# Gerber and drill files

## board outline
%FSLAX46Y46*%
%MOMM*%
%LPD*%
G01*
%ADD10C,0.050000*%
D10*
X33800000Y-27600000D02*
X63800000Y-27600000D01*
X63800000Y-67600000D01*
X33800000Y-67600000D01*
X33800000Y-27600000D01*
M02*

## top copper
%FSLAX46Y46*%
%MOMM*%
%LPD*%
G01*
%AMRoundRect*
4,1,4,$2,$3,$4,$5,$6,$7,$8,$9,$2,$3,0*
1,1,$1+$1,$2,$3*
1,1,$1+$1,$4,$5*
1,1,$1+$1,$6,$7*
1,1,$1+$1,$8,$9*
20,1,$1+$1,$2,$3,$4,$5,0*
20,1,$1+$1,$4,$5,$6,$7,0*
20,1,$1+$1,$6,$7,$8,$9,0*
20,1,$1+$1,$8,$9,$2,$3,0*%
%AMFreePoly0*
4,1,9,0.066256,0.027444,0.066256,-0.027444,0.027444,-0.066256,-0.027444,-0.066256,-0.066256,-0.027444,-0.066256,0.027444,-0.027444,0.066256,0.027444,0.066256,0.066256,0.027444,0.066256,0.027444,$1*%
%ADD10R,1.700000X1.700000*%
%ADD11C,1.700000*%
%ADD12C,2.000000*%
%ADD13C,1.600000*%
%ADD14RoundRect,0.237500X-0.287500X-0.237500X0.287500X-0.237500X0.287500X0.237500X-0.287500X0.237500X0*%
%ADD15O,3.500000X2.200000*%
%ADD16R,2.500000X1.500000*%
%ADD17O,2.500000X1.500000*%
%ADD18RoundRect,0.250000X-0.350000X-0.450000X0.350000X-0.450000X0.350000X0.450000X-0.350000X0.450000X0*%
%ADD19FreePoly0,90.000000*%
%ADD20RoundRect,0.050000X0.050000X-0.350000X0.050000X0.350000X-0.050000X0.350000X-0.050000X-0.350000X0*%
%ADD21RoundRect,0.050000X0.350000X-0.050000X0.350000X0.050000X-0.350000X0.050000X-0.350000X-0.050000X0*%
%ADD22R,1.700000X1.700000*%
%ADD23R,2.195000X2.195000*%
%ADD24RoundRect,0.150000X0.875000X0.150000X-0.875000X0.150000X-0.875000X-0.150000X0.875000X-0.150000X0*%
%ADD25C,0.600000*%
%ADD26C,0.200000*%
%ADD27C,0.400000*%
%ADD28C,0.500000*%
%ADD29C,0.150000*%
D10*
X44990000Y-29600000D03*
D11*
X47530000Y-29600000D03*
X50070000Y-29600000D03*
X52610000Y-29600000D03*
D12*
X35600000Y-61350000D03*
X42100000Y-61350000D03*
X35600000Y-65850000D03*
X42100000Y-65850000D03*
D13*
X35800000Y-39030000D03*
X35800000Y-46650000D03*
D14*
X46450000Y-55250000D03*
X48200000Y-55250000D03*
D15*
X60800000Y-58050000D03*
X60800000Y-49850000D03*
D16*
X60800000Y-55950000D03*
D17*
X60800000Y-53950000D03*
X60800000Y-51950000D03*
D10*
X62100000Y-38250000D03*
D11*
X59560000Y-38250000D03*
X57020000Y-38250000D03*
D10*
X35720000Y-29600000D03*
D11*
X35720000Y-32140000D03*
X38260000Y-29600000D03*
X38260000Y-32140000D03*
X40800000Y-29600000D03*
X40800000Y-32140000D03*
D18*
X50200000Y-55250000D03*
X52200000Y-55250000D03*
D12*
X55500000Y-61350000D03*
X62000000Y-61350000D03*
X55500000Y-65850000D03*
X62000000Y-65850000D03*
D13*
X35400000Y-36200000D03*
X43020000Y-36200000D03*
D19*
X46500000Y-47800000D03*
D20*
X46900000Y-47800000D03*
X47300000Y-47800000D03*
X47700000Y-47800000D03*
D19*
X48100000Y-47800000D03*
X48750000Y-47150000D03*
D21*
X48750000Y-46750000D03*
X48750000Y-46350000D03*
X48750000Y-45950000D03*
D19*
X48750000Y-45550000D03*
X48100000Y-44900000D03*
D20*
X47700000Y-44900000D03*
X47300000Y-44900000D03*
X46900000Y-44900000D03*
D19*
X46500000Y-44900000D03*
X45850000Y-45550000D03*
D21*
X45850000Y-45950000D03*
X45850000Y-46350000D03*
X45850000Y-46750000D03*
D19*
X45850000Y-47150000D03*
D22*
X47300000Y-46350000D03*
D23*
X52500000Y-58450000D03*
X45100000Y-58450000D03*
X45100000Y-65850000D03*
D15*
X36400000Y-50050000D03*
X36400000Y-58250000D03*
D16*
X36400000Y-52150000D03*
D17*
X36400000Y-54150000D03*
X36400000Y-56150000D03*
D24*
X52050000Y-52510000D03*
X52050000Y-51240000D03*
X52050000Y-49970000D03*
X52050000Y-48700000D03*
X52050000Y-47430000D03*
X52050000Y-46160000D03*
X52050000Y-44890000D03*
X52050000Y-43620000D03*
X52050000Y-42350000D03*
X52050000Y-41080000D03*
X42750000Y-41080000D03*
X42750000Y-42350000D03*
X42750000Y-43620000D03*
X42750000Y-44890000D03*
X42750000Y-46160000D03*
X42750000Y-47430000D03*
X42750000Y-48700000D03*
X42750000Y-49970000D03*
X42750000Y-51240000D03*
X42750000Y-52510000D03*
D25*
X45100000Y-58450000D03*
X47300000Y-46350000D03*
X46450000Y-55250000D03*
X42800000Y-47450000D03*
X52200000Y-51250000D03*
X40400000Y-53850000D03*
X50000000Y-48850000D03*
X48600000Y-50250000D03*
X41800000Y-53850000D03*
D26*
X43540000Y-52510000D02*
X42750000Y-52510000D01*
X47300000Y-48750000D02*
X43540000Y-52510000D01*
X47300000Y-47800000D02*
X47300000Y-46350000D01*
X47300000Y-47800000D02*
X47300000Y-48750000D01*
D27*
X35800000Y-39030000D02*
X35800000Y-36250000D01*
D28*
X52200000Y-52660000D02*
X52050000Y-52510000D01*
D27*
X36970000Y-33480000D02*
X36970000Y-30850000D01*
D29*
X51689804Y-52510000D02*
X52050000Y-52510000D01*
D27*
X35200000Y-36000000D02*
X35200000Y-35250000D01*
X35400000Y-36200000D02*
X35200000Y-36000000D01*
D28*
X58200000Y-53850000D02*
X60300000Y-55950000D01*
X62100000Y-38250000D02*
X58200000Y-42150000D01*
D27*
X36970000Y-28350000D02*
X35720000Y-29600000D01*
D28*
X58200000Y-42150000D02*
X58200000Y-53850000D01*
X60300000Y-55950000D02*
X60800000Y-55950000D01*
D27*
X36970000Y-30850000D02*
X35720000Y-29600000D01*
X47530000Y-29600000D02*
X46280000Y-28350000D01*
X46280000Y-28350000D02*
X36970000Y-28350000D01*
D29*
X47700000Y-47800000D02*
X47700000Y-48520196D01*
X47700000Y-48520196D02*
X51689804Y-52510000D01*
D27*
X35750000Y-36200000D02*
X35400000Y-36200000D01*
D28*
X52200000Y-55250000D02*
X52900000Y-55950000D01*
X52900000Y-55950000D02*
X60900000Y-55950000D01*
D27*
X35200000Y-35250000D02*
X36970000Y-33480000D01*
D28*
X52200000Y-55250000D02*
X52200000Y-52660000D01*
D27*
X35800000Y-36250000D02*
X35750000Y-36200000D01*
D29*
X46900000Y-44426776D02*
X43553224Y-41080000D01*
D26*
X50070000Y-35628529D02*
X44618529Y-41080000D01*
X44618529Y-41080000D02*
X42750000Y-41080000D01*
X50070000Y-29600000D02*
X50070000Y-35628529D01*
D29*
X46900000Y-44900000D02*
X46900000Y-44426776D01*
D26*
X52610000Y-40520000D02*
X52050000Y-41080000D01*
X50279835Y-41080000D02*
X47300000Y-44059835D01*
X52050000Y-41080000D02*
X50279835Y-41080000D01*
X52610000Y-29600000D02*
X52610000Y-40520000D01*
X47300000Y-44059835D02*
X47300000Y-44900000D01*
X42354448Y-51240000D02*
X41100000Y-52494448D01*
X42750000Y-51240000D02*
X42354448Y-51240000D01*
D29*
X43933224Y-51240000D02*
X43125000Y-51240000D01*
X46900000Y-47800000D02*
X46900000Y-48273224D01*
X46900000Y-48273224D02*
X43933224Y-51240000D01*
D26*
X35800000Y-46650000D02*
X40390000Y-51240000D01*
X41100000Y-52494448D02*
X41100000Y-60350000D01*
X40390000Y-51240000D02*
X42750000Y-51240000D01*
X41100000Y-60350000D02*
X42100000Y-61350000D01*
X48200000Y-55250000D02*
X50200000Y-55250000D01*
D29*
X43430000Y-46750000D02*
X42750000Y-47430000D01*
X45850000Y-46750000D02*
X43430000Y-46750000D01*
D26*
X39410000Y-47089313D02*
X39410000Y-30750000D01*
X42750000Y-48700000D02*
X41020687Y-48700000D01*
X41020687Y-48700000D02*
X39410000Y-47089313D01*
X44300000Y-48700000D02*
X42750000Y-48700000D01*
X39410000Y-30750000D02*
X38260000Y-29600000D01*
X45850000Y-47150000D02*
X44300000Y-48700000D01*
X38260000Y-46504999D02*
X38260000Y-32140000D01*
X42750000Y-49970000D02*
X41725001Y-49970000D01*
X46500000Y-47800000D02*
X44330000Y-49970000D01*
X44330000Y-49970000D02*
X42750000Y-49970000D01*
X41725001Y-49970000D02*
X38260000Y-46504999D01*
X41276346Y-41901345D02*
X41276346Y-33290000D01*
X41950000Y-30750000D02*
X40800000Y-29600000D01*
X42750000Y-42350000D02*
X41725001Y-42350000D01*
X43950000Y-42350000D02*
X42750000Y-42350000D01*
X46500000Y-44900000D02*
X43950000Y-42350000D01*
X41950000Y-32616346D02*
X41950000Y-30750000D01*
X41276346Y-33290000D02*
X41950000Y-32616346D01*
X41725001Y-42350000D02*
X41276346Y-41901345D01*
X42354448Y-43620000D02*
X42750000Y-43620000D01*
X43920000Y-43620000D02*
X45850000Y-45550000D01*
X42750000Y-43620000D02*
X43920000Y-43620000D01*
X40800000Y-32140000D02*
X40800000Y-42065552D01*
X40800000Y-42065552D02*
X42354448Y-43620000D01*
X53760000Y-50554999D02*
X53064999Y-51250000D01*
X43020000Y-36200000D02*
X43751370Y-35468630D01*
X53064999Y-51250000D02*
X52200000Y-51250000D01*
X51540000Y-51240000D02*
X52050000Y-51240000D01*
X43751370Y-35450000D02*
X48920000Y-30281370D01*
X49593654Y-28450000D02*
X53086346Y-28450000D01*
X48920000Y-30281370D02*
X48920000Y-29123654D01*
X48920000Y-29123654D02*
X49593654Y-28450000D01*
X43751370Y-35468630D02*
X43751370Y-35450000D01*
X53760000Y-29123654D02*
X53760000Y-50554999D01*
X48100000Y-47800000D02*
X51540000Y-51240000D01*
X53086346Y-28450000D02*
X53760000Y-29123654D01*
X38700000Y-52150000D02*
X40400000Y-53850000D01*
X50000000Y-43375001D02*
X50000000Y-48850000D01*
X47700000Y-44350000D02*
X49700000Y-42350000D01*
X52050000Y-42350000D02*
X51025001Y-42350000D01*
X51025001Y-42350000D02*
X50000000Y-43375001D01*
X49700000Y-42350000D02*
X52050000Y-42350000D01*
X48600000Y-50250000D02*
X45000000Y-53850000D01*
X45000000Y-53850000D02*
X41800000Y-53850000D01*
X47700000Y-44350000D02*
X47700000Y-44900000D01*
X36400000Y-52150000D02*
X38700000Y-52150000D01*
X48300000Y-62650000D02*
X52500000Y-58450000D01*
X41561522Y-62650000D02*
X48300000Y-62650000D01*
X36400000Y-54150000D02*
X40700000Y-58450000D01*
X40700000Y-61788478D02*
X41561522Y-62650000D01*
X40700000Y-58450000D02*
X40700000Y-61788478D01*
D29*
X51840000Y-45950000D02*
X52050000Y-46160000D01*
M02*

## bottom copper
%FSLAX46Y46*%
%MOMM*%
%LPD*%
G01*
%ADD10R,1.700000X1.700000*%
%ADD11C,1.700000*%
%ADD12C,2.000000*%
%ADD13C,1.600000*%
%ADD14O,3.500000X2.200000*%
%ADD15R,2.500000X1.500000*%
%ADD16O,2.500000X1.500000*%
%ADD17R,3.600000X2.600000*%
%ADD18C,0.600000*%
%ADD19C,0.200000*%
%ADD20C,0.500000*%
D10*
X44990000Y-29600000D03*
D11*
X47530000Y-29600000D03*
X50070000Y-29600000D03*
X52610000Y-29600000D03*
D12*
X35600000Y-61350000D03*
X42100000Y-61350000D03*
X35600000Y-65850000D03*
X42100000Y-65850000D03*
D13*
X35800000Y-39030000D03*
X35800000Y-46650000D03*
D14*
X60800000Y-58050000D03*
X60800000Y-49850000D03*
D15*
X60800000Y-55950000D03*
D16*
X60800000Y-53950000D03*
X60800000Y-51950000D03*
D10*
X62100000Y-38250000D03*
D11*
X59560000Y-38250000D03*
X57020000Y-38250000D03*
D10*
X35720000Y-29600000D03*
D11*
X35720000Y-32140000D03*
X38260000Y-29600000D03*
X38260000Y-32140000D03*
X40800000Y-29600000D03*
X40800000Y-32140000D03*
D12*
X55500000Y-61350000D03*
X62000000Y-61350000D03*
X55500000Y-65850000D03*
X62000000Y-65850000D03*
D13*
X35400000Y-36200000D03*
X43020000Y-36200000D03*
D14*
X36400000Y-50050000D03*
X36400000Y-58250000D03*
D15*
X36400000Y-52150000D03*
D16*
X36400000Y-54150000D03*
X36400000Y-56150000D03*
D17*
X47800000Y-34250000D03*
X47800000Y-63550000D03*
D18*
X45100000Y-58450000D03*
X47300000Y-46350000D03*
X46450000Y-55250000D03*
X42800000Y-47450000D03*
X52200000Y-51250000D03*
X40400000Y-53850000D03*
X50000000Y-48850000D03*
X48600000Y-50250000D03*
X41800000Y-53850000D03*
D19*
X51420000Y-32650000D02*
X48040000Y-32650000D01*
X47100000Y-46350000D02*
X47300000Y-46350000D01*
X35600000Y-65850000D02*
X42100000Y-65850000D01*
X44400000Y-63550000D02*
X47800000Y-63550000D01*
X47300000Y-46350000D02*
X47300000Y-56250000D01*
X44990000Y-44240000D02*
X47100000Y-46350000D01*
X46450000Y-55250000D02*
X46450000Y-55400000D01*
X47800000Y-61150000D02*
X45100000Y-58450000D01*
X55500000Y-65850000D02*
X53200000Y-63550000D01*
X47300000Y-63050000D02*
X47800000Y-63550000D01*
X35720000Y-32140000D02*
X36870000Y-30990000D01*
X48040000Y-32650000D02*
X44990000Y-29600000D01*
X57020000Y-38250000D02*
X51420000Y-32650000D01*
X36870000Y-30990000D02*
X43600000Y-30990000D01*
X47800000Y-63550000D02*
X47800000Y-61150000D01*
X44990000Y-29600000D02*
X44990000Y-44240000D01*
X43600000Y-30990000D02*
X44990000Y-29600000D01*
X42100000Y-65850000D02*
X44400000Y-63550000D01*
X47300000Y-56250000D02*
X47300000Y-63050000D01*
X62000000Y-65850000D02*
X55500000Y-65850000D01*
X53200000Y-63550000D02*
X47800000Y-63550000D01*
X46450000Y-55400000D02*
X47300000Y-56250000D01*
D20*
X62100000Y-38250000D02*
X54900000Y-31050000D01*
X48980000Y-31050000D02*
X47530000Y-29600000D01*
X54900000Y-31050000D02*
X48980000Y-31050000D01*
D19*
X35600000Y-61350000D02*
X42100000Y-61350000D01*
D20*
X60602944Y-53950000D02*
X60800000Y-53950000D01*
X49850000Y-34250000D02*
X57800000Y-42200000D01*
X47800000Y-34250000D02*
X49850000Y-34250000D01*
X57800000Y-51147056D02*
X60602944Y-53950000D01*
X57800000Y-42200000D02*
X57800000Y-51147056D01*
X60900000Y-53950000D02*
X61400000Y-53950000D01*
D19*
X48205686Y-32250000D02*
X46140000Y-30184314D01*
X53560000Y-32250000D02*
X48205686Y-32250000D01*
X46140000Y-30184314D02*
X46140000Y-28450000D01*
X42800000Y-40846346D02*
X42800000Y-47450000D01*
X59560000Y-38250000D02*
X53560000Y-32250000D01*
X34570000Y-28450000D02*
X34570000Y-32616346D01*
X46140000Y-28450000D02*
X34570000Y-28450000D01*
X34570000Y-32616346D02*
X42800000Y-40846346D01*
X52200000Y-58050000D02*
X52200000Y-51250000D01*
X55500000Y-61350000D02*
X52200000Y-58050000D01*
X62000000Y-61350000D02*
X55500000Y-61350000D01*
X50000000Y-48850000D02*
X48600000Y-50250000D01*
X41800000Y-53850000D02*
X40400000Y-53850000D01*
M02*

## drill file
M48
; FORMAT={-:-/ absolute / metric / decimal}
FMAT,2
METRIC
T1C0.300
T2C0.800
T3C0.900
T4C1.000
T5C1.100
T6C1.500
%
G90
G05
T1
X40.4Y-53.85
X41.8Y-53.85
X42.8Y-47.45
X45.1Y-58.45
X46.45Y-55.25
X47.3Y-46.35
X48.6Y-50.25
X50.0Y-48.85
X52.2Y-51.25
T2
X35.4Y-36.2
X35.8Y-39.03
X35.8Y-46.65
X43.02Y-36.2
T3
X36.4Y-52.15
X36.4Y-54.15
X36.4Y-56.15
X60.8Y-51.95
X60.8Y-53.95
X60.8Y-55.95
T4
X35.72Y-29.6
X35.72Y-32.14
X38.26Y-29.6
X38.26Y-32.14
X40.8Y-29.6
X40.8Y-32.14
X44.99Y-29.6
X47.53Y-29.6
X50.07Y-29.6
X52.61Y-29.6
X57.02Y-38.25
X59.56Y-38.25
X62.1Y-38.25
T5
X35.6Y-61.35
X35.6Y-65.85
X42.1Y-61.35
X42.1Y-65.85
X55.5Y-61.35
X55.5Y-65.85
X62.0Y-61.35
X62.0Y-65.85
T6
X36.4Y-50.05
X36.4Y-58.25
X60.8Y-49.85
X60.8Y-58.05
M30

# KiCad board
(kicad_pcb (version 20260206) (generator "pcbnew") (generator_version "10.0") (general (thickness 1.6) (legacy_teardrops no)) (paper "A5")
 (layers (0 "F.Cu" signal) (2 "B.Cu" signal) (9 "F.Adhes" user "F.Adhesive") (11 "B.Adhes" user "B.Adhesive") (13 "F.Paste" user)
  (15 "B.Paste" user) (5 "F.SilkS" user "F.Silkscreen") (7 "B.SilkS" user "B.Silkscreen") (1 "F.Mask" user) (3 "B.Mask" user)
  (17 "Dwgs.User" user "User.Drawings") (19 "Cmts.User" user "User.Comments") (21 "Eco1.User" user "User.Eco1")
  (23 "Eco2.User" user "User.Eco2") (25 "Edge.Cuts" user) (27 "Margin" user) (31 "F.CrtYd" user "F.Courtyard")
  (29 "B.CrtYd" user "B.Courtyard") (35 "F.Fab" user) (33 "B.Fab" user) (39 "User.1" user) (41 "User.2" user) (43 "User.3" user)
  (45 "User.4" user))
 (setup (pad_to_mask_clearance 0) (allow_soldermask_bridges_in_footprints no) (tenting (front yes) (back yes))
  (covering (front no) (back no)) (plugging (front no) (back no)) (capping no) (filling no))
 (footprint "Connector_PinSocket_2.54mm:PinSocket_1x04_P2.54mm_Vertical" (layer "F.Cu") (at 44.99 29.6 90)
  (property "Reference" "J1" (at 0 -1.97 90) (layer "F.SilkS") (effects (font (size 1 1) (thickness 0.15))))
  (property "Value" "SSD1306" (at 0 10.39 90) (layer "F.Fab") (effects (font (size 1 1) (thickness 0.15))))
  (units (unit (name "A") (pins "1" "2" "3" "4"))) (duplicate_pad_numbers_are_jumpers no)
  (pad "1" thru_hole rect (at 0 0 90) (size 1.7 1.7) (drill 1) (layers "*.Cu" "*.Mask") (remove_unused_layers no) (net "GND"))
  (pad "2" thru_hole circle (at 0 2.54 90) (size 1.7 1.7) (drill 1) (layers "*.Cu" "*.Mask") (remove_unused_layers no) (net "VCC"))
  (pad "3" thru_hole circle (at 0 5.08 90) (size 1.7 1.7) (drill 1) (layers "*.Cu" "*.Mask") (remove_unused_layers no) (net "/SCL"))
  (pad "4" thru_hole circle (at 0 7.62 90) (size 1.7 1.7) (drill 1) (layers "*.Cu" "*.Mask") (remove_unused_layers no) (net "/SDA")))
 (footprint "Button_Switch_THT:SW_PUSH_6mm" (layer "F.Cu") (at 35.6 61.35)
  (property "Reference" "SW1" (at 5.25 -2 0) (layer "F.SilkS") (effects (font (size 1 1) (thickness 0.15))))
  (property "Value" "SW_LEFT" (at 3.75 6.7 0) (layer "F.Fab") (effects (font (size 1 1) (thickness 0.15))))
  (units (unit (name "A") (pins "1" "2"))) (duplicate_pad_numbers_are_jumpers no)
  (pad "1" thru_hole circle (at 0 0 90) (size 2 2) (drill 1.1) (layers "*.Cu" "*.Mask") (remove_unused_layers no) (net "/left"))
  (pad "1" thru_hole circle (at 6.5 0 90) (size 2 2) (drill 1.1) (layers "*.Cu" "*.Mask") (remove_unused_layers no) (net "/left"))
  (pad "2" thru_hole circle (at 0 4.5 90) (size 2 2) (drill 1.1) (layers "*.Cu" "*.Mask") (remove_unused_layers no) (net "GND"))
  (pad "2" thru_hole circle (at 6.5 4.5 90) (size 2 2) (drill 1.1) (layers "*.Cu" "*.Mask") (remove_unused_layers no) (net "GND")))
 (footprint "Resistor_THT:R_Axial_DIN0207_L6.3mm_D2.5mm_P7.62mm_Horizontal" (layer "F.Cu") (at 35.8 39.03 -90)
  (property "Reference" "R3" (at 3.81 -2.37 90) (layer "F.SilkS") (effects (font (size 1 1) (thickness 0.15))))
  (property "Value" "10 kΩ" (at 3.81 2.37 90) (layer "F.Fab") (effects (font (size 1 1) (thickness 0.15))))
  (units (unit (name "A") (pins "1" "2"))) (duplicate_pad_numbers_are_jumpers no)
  (pad "1" thru_hole circle (at 0 0 270) (size 1.6 1.6) (drill 0.8) (layers "*.Cu" "*.Mask") (remove_unused_layers no) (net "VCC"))
  (pad "2" thru_hole circle (at 7.62 0 270) (size 1.6 1.6) (drill 0.8) (layers "*.Cu" "*.Mask") (remove_unused_layers no) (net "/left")))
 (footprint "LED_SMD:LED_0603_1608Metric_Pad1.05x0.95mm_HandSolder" (layer "F.Cu") (at 47.325 55.25)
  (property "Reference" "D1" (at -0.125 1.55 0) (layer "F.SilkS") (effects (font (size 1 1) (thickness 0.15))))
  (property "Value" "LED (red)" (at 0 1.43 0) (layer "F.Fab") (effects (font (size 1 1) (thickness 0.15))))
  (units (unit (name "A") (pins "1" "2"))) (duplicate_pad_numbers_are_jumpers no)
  (pad "1" smd roundrect (at -0.875 0) (size 1.05 0.95) (layers "F.Cu" "F.Mask" "F.Paste") (roundrect_rratio 0.25) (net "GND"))
  (pad "2" smd roundrect (at 0.875 0) (size 1.05 0.95) (layers "F.Cu" "F.Mask" "F.Paste") (roundrect_rratio 0.25) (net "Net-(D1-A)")))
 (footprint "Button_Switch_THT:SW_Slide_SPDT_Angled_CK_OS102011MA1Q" (layer "F.Cu") (at 60.8 55.95 90)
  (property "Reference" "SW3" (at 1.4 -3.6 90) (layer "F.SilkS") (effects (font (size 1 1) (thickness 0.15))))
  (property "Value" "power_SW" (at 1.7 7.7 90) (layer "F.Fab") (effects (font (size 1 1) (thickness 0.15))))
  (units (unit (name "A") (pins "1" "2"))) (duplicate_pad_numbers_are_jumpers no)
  (pad "" thru_hole oval (at -2.1 0 90) (size 2.2 3.5) (drill 1.5) (layers "*.Cu" "*.Mask") (remove_unused_layers no))
  (pad "" thru_hole oval (at 6.1 0 90) (size 2.2 3.5) (drill 1.5) (layers "*.Cu" "*.Mask") (remove_unused_layers no))
  (pad "1" thru_hole rect (at 0 0 90) (size 1.5 2.5) (drill 0.9) (layers "*.Cu" "*.Mask") (remove_unused_layers no) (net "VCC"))
  (pad "2" thru_hole oval (at 2 0 90) (size 1.5 2.5) (drill 0.9) (layers "*.Cu" "*.Mask") (remove_unused_layers no) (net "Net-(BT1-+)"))
  (pad "3" thru_hole oval (at 4 0 90) (size 1.5 2.5) (drill 0.9) (layers "*.Cu" "*.Mask") (remove_unused_layers no)))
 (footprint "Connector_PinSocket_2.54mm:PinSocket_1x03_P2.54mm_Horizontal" (layer "F.Cu") (at 62.1 38.25 -90)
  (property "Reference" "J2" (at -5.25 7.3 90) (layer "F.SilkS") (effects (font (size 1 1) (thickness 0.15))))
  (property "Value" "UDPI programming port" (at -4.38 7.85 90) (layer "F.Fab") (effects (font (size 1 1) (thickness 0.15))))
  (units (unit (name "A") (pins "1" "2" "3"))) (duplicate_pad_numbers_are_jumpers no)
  (pad "1" thru_hole rect (at 0 0 270) (size 1.7 1.7) (drill 1) (layers "*.Cu" "*.Mask") (remove_unused_layers no) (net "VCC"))
  (pad "2" thru_hole circle (at 0 2.54 270) (size 1.7 1.7) (drill 1) (layers "*.Cu" "*.Mask") (remove_unused_layers no) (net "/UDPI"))
  (pad "3" thru_hole circle (at 0 5.08 270) (size 1.7 1.7) (drill 1) (layers "*.Cu" "*.Mask") (remove_unused_layers no) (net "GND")))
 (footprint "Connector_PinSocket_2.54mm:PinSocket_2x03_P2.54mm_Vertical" (layer "F.Cu") (at 35.72 29.6 90)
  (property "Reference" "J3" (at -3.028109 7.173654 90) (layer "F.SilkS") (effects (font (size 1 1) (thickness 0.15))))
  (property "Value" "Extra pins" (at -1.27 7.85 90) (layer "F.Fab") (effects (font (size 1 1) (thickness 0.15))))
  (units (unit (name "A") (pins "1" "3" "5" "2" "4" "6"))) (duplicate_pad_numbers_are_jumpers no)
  (pad "1" thru_hole rect (at 0 0 90) (size 1.7 1.7) (drill 1) (layers "*.Cu" "*.Mask") (remove_unused_layers no) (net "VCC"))
  (pad "2" thru_hole circle (at -2.54 0 90) (size 1.7 1.7) (drill 1) (layers "*.Cu" "*.Mask") (remove_unused_layers no) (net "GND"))
  (pad "3" thru_hole circle (at 0 2.54 90) (size 1.7 1.7) (drill 1) (layers "*.Cu" "*.Mask") (remove_unused_layers no) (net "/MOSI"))
  (pad "4" thru_hole circle (at -2.54 2.54 90) (size 1.7 1.7) (drill 1) (layers "*.Cu" "*.Mask") (remove_unused_layers no) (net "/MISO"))
  (pad "5" thru_hole circle (at 0 5.08 90) (size 1.7 1.7) (drill 1) (layers "*.Cu" "*.Mask") (remove_unused_layers no) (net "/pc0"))
  (pad "6" thru_hole circle (at -2.54 5.08 90) (size 1.7 1.7) (drill 1) (layers "*.Cu" "*.Mask") (remove_unused_layers no) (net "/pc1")))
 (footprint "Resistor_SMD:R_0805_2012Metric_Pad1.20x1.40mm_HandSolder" (layer "F.Cu") (at 51.2 55.25)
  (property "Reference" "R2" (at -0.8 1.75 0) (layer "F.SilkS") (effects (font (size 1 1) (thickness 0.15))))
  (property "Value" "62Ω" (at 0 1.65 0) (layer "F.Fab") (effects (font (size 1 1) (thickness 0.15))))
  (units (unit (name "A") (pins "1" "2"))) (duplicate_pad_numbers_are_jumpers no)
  (pad "1" smd roundrect (at -1 0) (size 1.2 1.4) (layers "F.Cu" "F.Mask" "F.Paste") (roundrect_rratio 0.208333) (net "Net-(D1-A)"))
  (pad "2" smd roundrect (at 1 0) (size 1.2 1.4) (layers "F.Cu" "F.Mask" "F.Paste") (roundrect_rratio 0.208333) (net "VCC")))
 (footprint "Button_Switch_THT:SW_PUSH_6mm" (layer "F.Cu") (at 55.5 61.35)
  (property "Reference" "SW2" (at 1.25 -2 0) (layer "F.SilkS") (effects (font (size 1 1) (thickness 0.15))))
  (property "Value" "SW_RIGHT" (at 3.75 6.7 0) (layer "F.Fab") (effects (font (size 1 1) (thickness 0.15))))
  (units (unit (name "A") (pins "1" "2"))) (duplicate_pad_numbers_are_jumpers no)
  (pad "1" thru_hole circle (at 0 0 90) (size 2 2) (drill 1.1) (layers "*.Cu" "*.Mask") (remove_unused_layers no) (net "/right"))
  (pad "1" thru_hole circle (at 6.5 0 90) (size 2 2) (drill 1.1) (layers "*.Cu" "*.Mask") (remove_unused_layers no) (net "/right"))
  (pad "2" thru_hole circle (at 0 4.5 90) (size 2 2) (drill 1.1) (layers "*.Cu" "*.Mask") (remove_unused_layers no) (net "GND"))
  (pad "2" thru_hole circle (at 6.5 4.5 90) (size 2 2) (drill 1.1) (layers "*.Cu" "*.Mask") (remove_unused_layers no) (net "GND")))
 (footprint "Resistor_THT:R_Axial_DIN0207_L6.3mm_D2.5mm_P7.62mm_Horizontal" (layer "F.Cu") (at 35.4 36.2)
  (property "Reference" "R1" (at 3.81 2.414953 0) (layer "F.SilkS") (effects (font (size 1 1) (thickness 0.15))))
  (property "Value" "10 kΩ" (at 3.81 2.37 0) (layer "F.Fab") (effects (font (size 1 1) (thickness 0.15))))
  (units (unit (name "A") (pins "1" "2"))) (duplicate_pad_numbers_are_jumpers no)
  (pad "1" thru_hole circle (at 0 0) (size 1.6 1.6) (drill 0.8) (layers "*.Cu" "*.Mask") (remove_unused_layers no) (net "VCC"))
  (pad "2" thru_hole circle (at 7.62 0) (size 1.6 1.6) (drill 0.8) (layers "*.Cu" "*.Mask") (remove_unused_layers no) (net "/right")))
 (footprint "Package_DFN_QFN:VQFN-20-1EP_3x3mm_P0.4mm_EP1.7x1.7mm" (layer "F.Cu") (at 47.3 46.35 90)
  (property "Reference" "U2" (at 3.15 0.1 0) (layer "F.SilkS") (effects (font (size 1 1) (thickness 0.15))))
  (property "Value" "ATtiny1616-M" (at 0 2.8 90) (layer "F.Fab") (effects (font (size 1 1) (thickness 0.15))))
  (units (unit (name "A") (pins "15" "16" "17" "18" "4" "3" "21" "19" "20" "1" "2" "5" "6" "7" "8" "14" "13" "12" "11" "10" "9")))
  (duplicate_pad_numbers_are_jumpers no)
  (pad "" smd roundrect (at -0.425 -0.425 90) (size 0.69 0.69) (layers "F.Paste") (roundrect_rratio 0.25))
  (pad "" smd roundrect (at -0.425 0.425 90) (size 0.69 0.69) (layers "F.Paste") (roundrect_rratio 0.25))
  (pad "" smd roundrect (at 0.425 -0.425 90) (size 0.69 0.69) (layers "F.Paste") (roundrect_rratio 0.25))
  (pad "" smd roundrect (at 0.425 0.425 90) (size 0.69 0.69) (layers "F.Paste") (roundrect_rratio 0.25))
  (pad "1" smd custom (at -1.45 -0.8 90) (size 0.143431 0.143431) (layers "F.Cu" "F.Mask" "F.Paste") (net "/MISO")
   (options (clearance outline) (anchor circle)) (primitives))
  (pad "2" smd roundrect (at -1.45 -0.4 90) (size 0.8 0.2) (layers "F.Cu" "F.Mask" "F.Paste") (roundrect_rratio 0.25) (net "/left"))
  (pad "3" smd roundrect (at -1.45 0 90) (size 0.8 0.2) (layers "F.Cu" "F.Mask" "F.Paste") (roundrect_rratio 0.25) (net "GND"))
  (pad "4" smd roundrect (at -1.45 0.4 90) (size 0.8 0.2) (layers "F.Cu" "F.Mask" "F.Paste") (roundrect_rratio 0.25) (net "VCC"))
  (pad "5" smd custom (at -1.45 0.8 90) (size 0.143431 0.143431) (layers "F.Cu" "F.Mask" "F.Paste") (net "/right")
   (options (clearance outline) (anchor circle)) (primitives))
  (pad "6" smd custom (at -0.8 1.45 90) (size 0.143431 0.143431) (layers "F.Cu" "F.Mask" "F.Paste") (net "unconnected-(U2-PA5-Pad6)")
   (options (clearance outline) (anchor circle)) (primitives))
  (pad "7" smd roundrect (at -0.4 1.45 90) (size 0.2 0.8) (layers "F.Cu" "F.Mask" "F.Paste") (roundrect_rratio 0.25)
   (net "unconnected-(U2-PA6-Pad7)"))
  (pad "8" smd roundrect (at 0 1.45 90) (size 0.2 0.8) (layers "F.Cu" "F.Mask" "F.Paste") (roundrect_rratio 0.25)
   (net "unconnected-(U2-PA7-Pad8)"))
  (pad "9" smd roundrect (at 0.4 1.45 90) (size 0.2 0.8) (layers "F.Cu" "F.Mask" "F.Paste") (roundrect_rratio 0.25)
   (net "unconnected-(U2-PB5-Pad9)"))
  (pad "10" smd custom (at 0.8 1.45 90) (size 0.143431 0.143431) (layers "F.Cu" "F.Mask" "F.Paste") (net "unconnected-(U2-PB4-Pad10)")
   (options (clearance outline) (anchor circle)) (primitives))
  (pad "11" smd custom (at 1.45 0.8 90) (size 0.143431 0.143431) (layers "F.Cu" "F.Mask" "F.Paste") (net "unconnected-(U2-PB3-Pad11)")
   (options (clearance outline) (anchor circle)) (primitives))
  (pad "12" smd roundrect (at 1.45 0.4 90) (size 0.8 0.2) (layers "F.Cu" "F.Mask" "F.Paste") (roundrect_rratio 0.25) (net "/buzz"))
  (pad "13" smd roundrect (at 1.45 0 90) (size 0.8 0.2) (layers "F.Cu" "F.Mask" "F.Paste") (roundrect_rratio 0.25) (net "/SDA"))
  (pad "14" smd roundrect (at 1.45 -0.4 90) (size 0.8 0.2) (layers "F.Cu" "F.Mask" "F.Paste") (roundrect_rratio 0.25) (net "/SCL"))
  (pad "15" smd custom (at 1.45 -0.8 90) (size 0.143431 0.143431) (layers "F.Cu" "F.Mask" "F.Paste") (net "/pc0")
   (options (clearance outline) (anchor circle)) (primitives))
  (pad "16" smd custom (at 0.8 -1.45 90) (size 0.143431 0.143431) (layers "F.Cu" "F.Mask" "F.Paste") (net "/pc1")
   (options (clearance outline) (anchor circle)) (primitives))
  (pad "17" smd roundrect (at 0.4 -1.45 90) (size 0.2 0.8) (layers "F.Cu" "F.Mask" "F.Paste") (roundrect_rratio 0.25)
   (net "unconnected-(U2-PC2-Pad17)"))
  (pad "18" smd roundrect (at 0 -1.45 90) (size 0.2 0.8) (layers "F.Cu" "F.Mask" "F.Paste") (roundrect_rratio 0.25)
   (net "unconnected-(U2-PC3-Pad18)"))
  (pad "19" smd roundrect (at -0.4 -1.45 90) (size 0.2 0.8) (layers "F.Cu" "F.Mask" "F.Paste") (roundrect_rratio 0.25) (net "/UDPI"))
  (pad "20" smd custom (at -0.8 -1.45 90) (size 0.143431 0.143431) (layers "F.Cu" "F.Mask" "F.Paste") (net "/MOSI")
   (options (clearance outline) (anchor circle)) (primitives))
  (pad "21" smd rect (at 0 0 90) (size 1.7 1.7) (layers "F.Cu" "F.Mask") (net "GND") (zone_connect 2)))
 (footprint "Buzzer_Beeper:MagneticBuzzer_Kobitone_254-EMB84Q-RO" (layer "F.Cu") (at 48.8 62.15 -90)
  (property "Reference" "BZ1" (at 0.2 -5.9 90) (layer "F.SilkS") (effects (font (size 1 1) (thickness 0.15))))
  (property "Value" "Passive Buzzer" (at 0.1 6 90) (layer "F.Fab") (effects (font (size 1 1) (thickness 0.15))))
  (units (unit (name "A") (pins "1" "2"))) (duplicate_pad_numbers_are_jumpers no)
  (pad "1" smd rect (at -3.7 -3.7 180) (size 2.195 2.195) (layers "F.Cu" "F.Mask" "F.Paste") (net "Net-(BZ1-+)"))
  (pad "2" smd rect (at -3.7 3.7 180) (size 2.195 2.195) (layers "F.Cu" "F.Mask" "F.Paste") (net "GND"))
  (pad "3" smd rect (at 3.7 3.7 180) (size 2.195 2.195) (layers "F.Cu" "F.Mask" "F.Paste")))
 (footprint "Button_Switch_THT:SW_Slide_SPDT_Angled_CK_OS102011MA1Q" (layer "F.Cu") (at 36.4 52.15 -90)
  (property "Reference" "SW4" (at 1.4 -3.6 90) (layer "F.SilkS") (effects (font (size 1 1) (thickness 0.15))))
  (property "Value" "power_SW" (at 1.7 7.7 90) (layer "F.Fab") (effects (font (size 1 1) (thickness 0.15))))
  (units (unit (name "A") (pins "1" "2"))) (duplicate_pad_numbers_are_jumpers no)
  (pad "" thru_hole oval (at -2.1 0 270) (size 2.2 3.5) (drill 1.5) (layers "*.Cu" "*.Mask") (remove_unused_layers no))
  (pad "" thru_hole oval (at 6.1 0 270) (size 2.2 3.5) (drill 1.5) (layers "*.Cu" "*.Mask") (remove_unused_layers no))
  (pad "1" thru_hole rect (at 0 0 270) (size 1.5 2.5) (drill 0.9) (layers "*.Cu" "*.Mask") (remove_unused_layers no) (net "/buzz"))
  (pad "2" thru_hole oval (at 2 0 270) (size 1.5 2.5) (drill 0.9) (layers "*.Cu" "*.Mask") (remove_unused_layers no) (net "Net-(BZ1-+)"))
  (pad "3" thru_hole oval (at 4 0 270) (size 1.5 2.5) (drill 0.9) (layers "*.Cu" "*.Mask") (remove_unused_layers no)))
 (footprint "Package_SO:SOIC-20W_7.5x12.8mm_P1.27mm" (layer "F.Cu") (at 47.4 46.795 180)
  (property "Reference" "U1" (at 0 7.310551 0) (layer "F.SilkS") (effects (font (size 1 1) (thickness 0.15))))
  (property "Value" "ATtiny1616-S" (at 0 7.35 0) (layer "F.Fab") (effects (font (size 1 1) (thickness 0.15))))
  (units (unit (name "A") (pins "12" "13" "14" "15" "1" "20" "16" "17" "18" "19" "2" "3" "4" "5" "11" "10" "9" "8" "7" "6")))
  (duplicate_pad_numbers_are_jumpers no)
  (pad "1" smd roundrect (at -4.65 -5.715 180) (size 2.05 0.6) (layers "F.Cu" "F.Mask" "F.Paste") (roundrect_rratio 0.25) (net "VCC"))
  (pad "2" smd roundrect (at -4.65 -4.445 180) (size 2.05 0.6) (layers "F.Cu" "F.Mask" "F.Paste") (roundrect_rratio 0.25) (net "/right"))
  (pad "3" smd roundrect (at -4.65 -3.175 180) (size 2.05 0.6) (layers "F.Cu" "F.Mask" "F.Paste") (roundrect_rratio 0.25)
   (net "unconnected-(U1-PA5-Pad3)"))
  (pad "4" smd roundrect (at -4.65 -1.905 180) (size 2.05 0.6) (layers "F.Cu" "F.Mask" "F.Paste") (roundrect_rratio 0.25)
   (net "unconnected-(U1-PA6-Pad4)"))
  (pad "5" smd roundrect (at -4.65 -0.635 180) (size 2.05 0.6) (layers "F.Cu" "F.Mask" "F.Paste") (roundrect_rratio 0.25)
   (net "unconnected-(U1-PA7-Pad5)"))
  (pad "6" smd roundrect (at -4.65 0.635 180) (size 2.05 0.6) (layers "F.Cu" "F.Mask" "F.Paste") (roundrect_rratio 0.25)
   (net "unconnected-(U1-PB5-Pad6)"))
  (pad "7" smd roundrect (at -4.65 1.905 180) (size 2.05 0.6) (layers "F.Cu" "F.Mask" "F.Paste") (roundrect_rratio 0.25)
   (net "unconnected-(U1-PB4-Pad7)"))
  (pad "8" smd roundrect (at -4.65 3.175 180) (size 2.05 0.6) (layers "F.Cu" "F.Mask" "F.Paste") (roundrect_rratio 0.25)
   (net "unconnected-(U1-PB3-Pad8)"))
  (pad "9" smd roundrect (at -4.65 4.445 180) (size 2.05 0.6) (layers "F.Cu" "F.Mask" "F.Paste") (roundrect_rratio 0.25) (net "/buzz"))
  (pad "10" smd roundrect (at -4.65 5.715 180) (size 2.05 0.6) (layers "F.Cu" "F.Mask" "F.Paste") (roundrect_rratio 0.25) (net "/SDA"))
  (pad "11" smd roundrect (at 4.65 5.715 180) (size 2.05 0.6) (layers "F.Cu" "F.Mask" "F.Paste") (roundrect_rratio 0.25) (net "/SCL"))
  (pad "12" smd roundrect (at 4.65 4.445 180) (size 2.05 0.6) (layers "F.Cu" "F.Mask" "F.Paste") (roundrect_rratio 0.25) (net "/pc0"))
  (pad "13" smd roundrect (at 4.65 3.175 180) (size 2.05 0.6) (layers "F.Cu" "F.Mask" "F.Paste") (roundrect_rratio 0.25) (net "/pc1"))
  (pad "14" smd roundrect (at 4.65 1.905 180) (size 2.05 0.6) (layers "F.Cu" "F.Mask" "F.Paste") (roundrect_rratio 0.25)
   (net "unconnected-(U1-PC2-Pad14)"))
  (pad "15" smd roundrect (at 4.65 0.635 180) (size 2.05 0.6) (layers "F.Cu" "F.Mask" "F.Paste") (roundrect_rratio 0.25)
   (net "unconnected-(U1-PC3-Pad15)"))
  (pad "16" smd roundrect (at 4.65 -0.635 180) (size 2.05 0.6) (layers "F.Cu" "F.Mask" "F.Paste") (roundrect_rratio 0.25) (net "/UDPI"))
  (pad "17" smd roundrect (at 4.65 -1.905 180) (size 2.05 0.6) (layers "F.Cu" "F.Mask" "F.Paste") (roundrect_rratio 0.25) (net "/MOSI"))
  (pad "18" smd roundrect (at 4.65 -3.175 180) (size 2.05 0.6) (layers "F.Cu" "F.Mask" "F.Paste") (roundrect_rratio 0.25) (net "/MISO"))
  (pad "19" smd roundrect (at 4.65 -4.445 180) (size 2.05 0.6) (layers "F.Cu" "F.Mask" "F.Paste") (roundrect_rratio 0.25) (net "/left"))
  (pad "20" smd roundrect (at 4.65 -5.715 180) (size 2.05 0.6) (layers "F.Cu" "F.Mask" "F.Paste") (roundrect_rratio 0.25) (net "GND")))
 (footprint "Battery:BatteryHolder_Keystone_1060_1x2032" (layer "B.Cu") (at 47.8 48.9 -90)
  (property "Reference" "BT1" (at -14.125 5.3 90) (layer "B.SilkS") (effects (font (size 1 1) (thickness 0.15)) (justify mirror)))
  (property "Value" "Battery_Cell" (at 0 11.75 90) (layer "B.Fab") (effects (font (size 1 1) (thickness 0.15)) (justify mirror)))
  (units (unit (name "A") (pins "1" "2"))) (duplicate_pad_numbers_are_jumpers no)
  (pad "1" smd rect (at -14.65 0 90) (size 2.6 3.6) (layers "B.Cu" "B.Mask" "B.Paste") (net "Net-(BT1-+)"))
  (pad "2" smd rect (at 14.65 0 90) (size 2.6 3.6) (layers "B.Cu" "B.Mask" "B.Paste") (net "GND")))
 (gr_rect (start 33.8 27.6) (end 63.8 67.6) (stroke (width 0.05) (type solid)) (fill no) (layer "Edge.Cuts"))
 (segment (start 43.54 52.51) (end 42.75 52.51) (width 0.2) (layer "F.Cu") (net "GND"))
 (segment (start 47.3 48.75) (end 43.54 52.51) (width 0.2) (layer "F.Cu") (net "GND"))
 (segment (start 47.3 47.8) (end 47.3 46.35) (width 0.2) (layer "F.Cu") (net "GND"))
 (segment (start 47.3 47.8) (end 47.3 48.75) (width 0.2) (layer "F.Cu") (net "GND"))
 (via (at 45.1 58.45) (size 0.6) (drill 0.3) (layers "F.Cu" "B.Cu") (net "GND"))
 (via (at 47.3 46.35) (size 0.6) (drill 0.3) (layers "F.Cu" "B.Cu") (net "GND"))
 (via (at 46.45 55.25) (size 0.6) (drill 0.3) (layers "F.Cu" "B.Cu") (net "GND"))
 (segment (start 51.42 32.65) (end 48.04 32.65) (width 0.2) (layer "B.Cu") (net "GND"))
 (segment (start 47.1 46.35) (end 47.3 46.35) (width 0.2) (layer "B.Cu") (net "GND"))
 (segment (start 35.6 65.85) (end 42.1 65.85) (width 0.2) (layer "B.Cu") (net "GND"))
 (segment (start 44.4 63.55) (end 47.8 63.55) (width 0.2) (layer "B.Cu") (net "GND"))
 (segment (start 47.3 46.35) (end 47.3 56.25) (width 0.2) (layer "B.Cu") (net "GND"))
 (segment (start 44.99 44.24) (end 47.1 46.35) (width 0.2) (layer "B.Cu") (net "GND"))
 (segment (start 46.45 55.25) (end 46.45 55.4) (width 0.2) (layer "B.Cu") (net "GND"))
 (segment (start 47.8 61.15) (end 45.1 58.45) (width 0.2) (layer "B.Cu") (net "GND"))
 (segment (start 55.5 65.85) (end 53.2 63.55) (width 0.2) (layer "B.Cu") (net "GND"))
 (segment (start 47.3 63.05) (end 47.8 63.55) (width 0.2) (layer "B.Cu") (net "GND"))
 (segment (start 35.72 32.14) (end 36.87 30.99) (width 0.2) (layer "B.Cu") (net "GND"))
 (segment (start 48.04 32.65) (end 44.99 29.6) (width 0.2) (layer "B.Cu") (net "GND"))
 (segment (start 57.02 38.25) (end 51.42 32.65) (width 0.2) (layer "B.Cu") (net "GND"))
 (segment (start 36.87 30.99) (end 43.6 30.99) (width 0.2) (layer "B.Cu") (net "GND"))
 (segment (start 47.8 63.55) (end 47.8 61.15) (width 0.2) (layer "B.Cu") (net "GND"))
 (segment (start 44.99 29.6) (end 44.99 44.24) (width 0.2) (layer "B.Cu") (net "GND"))
 (segment (start 43.6 30.99) (end 44.99 29.6) (width 0.2) (layer "B.Cu") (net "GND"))
 (segment (start 42.1 65.85) (end 44.4 63.55) (width 0.2) (layer "B.Cu") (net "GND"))
 (segment (start 47.3 56.25) (end 47.3 63.05) (width 0.2) (layer "B.Cu") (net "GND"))
 (segment (start 62 65.85) (end 55.5 65.85) (width 0.2) (layer "B.Cu") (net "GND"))
 (segment (start 53.2 63.55) (end 47.8 63.55) (width 0.2) (layer "B.Cu") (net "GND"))
 (segment (start 46.45 55.4) (end 47.3 56.25) (width 0.2) (layer "B.Cu") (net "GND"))
 (segment (start 35.8 39.03) (end 35.8 36.25) (width 0.4) (layer "F.Cu") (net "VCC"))
 (segment (start 52.2 52.66) (end 52.05 52.51) (width 0.5) (layer "F.Cu") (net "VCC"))
 (segment (start 36.97 33.48) (end 36.97 30.85) (width 0.4) (layer "F.Cu") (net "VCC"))
 (segment (start 51.689804 52.51) (end 52.05 52.51) (width 0.15) (layer "F.Cu") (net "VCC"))
 (segment (start 35.2 36) (end 35.2 35.25) (width 0.4) (layer "F.Cu") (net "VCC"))
 (segment (start 35.4 36.2) (end 35.2 36) (width 0.4) (layer "F.Cu") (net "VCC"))
 (segment (start 58.2 53.85) (end 60.3 55.95) (width 0.5) (layer "F.Cu") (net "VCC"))
 (segment (start 62.1 38.25) (end 58.2 42.15) (width 0.5) (layer "F.Cu") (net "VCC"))
 (segment (start 36.97 28.35) (end 35.72 29.6) (width 0.4) (layer "F.Cu") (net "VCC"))
 (segment (start 58.2 42.15) (end 58.2 53.85) (width 0.5) (layer "F.Cu") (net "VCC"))
 (segment (start 60.3 55.95) (end 60.8 55.95) (width 0.5) (layer "F.Cu") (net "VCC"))
 (segment (start 36.97 30.85) (end 35.72 29.6) (width 0.4) (layer "F.Cu") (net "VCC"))
 (segment (start 47.53 29.6) (end 46.28 28.35) (width 0.4) (layer "F.Cu") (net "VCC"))
 (segment (start 46.28 28.35) (end 36.97 28.35) (width 0.4) (layer "F.Cu") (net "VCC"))
 (segment (start 47.7 47.8) (end 47.7 48.520196) (width 0.15) (layer "F.Cu") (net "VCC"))
 (segment (start 47.7 48.520196) (end 51.689804 52.51) (width 0.15) (layer "F.Cu") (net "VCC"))
 (segment (start 35.75 36.2) (end 35.4 36.2) (width 0.4) (layer "F.Cu") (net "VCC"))
 (segment (start 52.2 55.25) (end 52.9 55.95) (width 0.5) (layer "F.Cu") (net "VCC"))
 (segment (start 52.9 55.95) (end 60.9 55.95) (width 0.5) (layer "F.Cu") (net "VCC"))
 (segment (start 35.2 35.25) (end 36.97 33.48) (width 0.4) (layer "F.Cu") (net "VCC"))
 (segment (start 52.2 55.25) (end 52.2 52.66) (width 0.5) (layer "F.Cu") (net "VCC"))
 (segment (start 35.8 36.25) (end 35.75 36.2) (width 0.4) (layer "F.Cu") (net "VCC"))
 (segment (start 62.1 38.25) (end 54.9 31.05) (width 0.5) (layer "B.Cu") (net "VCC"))
 (segment (start 48.98 31.05) (end 47.53 29.6) (width 0.5) (layer "B.Cu") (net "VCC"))
 (segment (start 54.9 31.05) (end 48.98 31.05) (width 0.5) (layer "B.Cu") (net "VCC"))
 (segment (start 46.9 44.426776) (end 43.553224 41.08) (width 0.15) (layer "F.Cu") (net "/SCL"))
 (segment (start 50.07 35.628529) (end 44.618529 41.08) (width 0.2) (layer "F.Cu") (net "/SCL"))
 (segment (start 44.618529 41.08) (end 42.75 41.08) (width 0.2) (layer "F.Cu") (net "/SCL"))
 (segment (start 50.07 29.6) (end 50.07 35.628529) (width 0.2) (layer "F.Cu") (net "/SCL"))
 (segment (start 46.9 44.9) (end 46.9 44.426776) (width 0.15) (layer "F.Cu") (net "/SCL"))
 (segment (start 52.61 40.52) (end 52.05 41.08) (width 0.2) (layer "F.Cu") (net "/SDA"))
 (segment (start 50.279835 41.08) (end 47.3 44.059835) (width 0.2) (layer "F.Cu") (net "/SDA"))
 (segment (start 52.05 41.08) (end 50.279835 41.08) (width 0.2) (layer "F.Cu") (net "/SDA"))
 (segment (start 52.61 29.6) (end 52.61 40.52) (width 0.2) (layer "F.Cu") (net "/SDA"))
 (segment (start 47.3 44.059835) (end 47.3 44.9) (width 0.2) (layer "F.Cu") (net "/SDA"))
 (segment (start 42.354448 51.24) (end 41.1 52.494448) (width 0.2) (layer "F.Cu") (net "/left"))
 (segment (start 42.75 51.24) (end 42.354448 51.24) (width 0.2) (layer "F.Cu") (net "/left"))
 (segment (start 43.933224 51.24) (end 43.125 51.24) (width 0.15) (layer "F.Cu") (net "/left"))
 (segment (start 46.9 47.8) (end 46.9 48.273224) (width 0.15) (layer "F.Cu") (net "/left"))
 (segment (start 46.9 48.273224) (end 43.933224 51.24) (width 0.15) (layer "F.Cu") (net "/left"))
 (segment (start 35.8 46.65) (end 40.39 51.24) (width 0.2) (layer "F.Cu") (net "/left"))
 (segment (start 41.1 52.494448) (end 41.1 60.35) (width 0.2) (layer "F.Cu") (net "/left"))
 (segment (start 40.39 51.24) (end 42.75 51.24) (width 0.2) (layer "F.Cu") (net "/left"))
 (segment (start 41.1 60.35) (end 42.1 61.35) (width 0.2) (layer "F.Cu") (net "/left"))
 (segment (start 35.6 61.35) (end 42.1 61.35) (width 0.2) (layer "B.Cu") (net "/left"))
 (segment (start 48.2 55.25) (end 50.2 55.25) (width 0.2) (layer "F.Cu") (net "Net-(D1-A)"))
 (segment (start 60.602944 53.95) (end 60.8 53.95) (width 0.5) (layer "B.Cu") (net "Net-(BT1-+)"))
 (segment (start 49.85 34.25) (end 57.8 42.2) (width 0.5) (layer "B.Cu") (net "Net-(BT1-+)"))
 (segment (start 47.8 34.25) (end 49.85 34.25) (width 0.5) (layer "B.Cu") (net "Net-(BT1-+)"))
 (segment (start 57.8 51.147056) (end 60.602944 53.95) (width 0.5) (layer "B.Cu") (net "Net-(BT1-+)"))
 (segment (start 57.8 42.2) (end 57.8 51.147056) (width 0.5) (layer "B.Cu") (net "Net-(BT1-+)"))
 (segment (start 60.9 53.95) (end 61.4 53.95) (width 0.5) (layer "B.Cu") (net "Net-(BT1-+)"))
 (segment (start 43.43 46.75) (end 42.75 47.43) (width 0.15) (layer "F.Cu") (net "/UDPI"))
 (segment (start 45.85 46.75) (end 43.43 46.75) (width 0.15) (layer "F.Cu") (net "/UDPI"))
 (via (at 42.8 47.45) (size 0.6) (drill 0.3) (layers "F.Cu" "B.Cu") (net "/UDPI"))
 (segment (start 48.205686 32.25) (end 46.14 30.184314) (width 0.2) (layer "B.Cu") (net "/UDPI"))
 (segment (start 53.56 32.25) (end 48.205686 32.25) (width 0.2) (layer "B.Cu") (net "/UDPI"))
 (segment (start 46.14 30.184314) (end 46.14 28.45) (width 0.2) (layer "B.Cu") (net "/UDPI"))
 (segment (start 42.8 40.846346) (end 42.8 47.45) (width 0.2) (layer "B.Cu") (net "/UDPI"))
 (segment (start 59.56 38.25) (end 53.56 32.25) (width 0.2) (layer "B.Cu") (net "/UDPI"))
 (segment (start 34.57 28.45) (end 34.57 32.616346) (width 0.2) (layer "B.Cu") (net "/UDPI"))
 (segment (start 46.14 28.45) (end 34.57 28.45) (width 0.2) (layer "B.Cu") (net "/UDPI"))
 (segment (start 34.57 32.616346) (end 42.8 40.846346) (width 0.2) (layer "B.Cu") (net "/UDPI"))
 (segment (start 39.41 47.089313) (end 39.41 30.75) (width 0.2) (layer "F.Cu") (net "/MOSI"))
 (segment (start 42.75 48.7) (end 41.020687 48.7) (width 0.2) (layer "F.Cu") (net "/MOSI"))
 (segment (start 41.020687 48.7) (end 39.41 47.089313) (width 0.2) (layer "F.Cu") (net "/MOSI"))
 (segment (start 44.3 48.7) (end 42.75 48.7) (width 0.2) (layer "F.Cu") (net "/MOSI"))
 (segment (start 39.41 30.75) (end 38.26 29.6) (width 0.2) (layer "F.Cu") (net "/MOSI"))
 (segment (start 45.85 47.15) (end 44.3 48.7) (width 0.2) (layer "F.Cu") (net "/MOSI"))
 (segment (start 38.26 46.504999) (end 38.26 32.14) (width 0.2) (layer "F.Cu") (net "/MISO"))
 (segment (start 42.75 49.97) (end 41.725001 49.97) (width 0.2) (layer "F.Cu") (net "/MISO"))
 (segment (start 46.5 47.8) (end 44.33 49.97) (width 0.2) (layer "F.Cu") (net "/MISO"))
 (segment (start 44.33 49.97) (end 42.75 49.97) (width 0.2) (layer "F.Cu") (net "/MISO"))
 (segment (start 41.725001 49.97) (end 38.26 46.504999) (width 0.2) (layer "F.Cu") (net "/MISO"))
 (segment (start 41.276346 41.901345) (end 41.276346 33.29) (width 0.2) (layer "F.Cu") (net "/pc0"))
 (segment (start 41.95 30.75) (end 40.8 29.6) (width 0.2) (layer "F.Cu") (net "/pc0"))
 (segment (start 42.75 42.35) (end 41.725001 42.35) (width 0.2) (layer "F.Cu") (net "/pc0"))
 (segment (start 43.95 42.35) (end 42.75 42.35) (width 0.2) (layer "F.Cu") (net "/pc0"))
 (segment (start 46.5 44.9) (end 43.95 42.35) (width 0.2) (layer "F.Cu") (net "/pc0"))
 (segment (start 41.95 32.616346) (end 41.95 30.75) (width 0.2) (layer "F.Cu") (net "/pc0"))
 (segment (start 41.276346 33.29) (end 41.95 32.616346) (width 0.2) (layer "F.Cu") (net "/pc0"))
 (segment (start 41.725001 42.35) (end 41.276346 41.901345) (width 0.2) (layer "F.Cu") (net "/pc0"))
 (segment (start 42.354448 43.62) (end 42.75 43.62) (width 0.2) (layer "F.Cu") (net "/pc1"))
 (segment (start 43.92 43.62) (end 45.85 45.55) (width 0.2) (layer "F.Cu") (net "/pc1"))
 (segment (start 42.75 43.62) (end 43.92 43.62) (width 0.2) (layer "F.Cu") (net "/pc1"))
 (segment (start 40.8 32.14) (end 40.8 42.065552) (width 0.2) (layer "F.Cu") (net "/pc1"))
 (segment (start 40.8 42.065552) (end 42.354448 43.62) (width 0.2) (layer "F.Cu") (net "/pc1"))
 (segment (start 53.76 50.554999) (end 53.064999 51.25) (width 0.2) (layer "F.Cu") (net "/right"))
 (segment (start 43.02 36.2) (end 43.75137 35.46863) (width 0.2) (layer "F.Cu") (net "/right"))
 (segment (start 53.064999 51.25) (end 52.2 51.25) (width 0.2) (layer "F.Cu") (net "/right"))
 (segment (start 51.54 51.24) (end 52.05 51.24) (width 0.2) (layer "F.Cu") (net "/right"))
 (segment (start 43.75137 35.45) (end 48.92 30.28137) (width 0.2) (layer "F.Cu") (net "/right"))
 (segment (start 49.593654 28.45) (end 53.086346 28.45) (width 0.2) (layer "F.Cu") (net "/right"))
 (segment (start 48.92 30.28137) (end 48.92 29.123654) (width 0.2) (layer "F.Cu") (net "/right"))
 (segment (start 48.92 29.123654) (end 49.593654 28.45) (width 0.2) (layer "F.Cu") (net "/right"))
 (segment (start 43.75137 35.46863) (end 43.75137 35.45) (width 0.2) (layer "F.Cu") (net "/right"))
 (segment (start 53.76 29.123654) (end 53.76 50.554999) (width 0.2) (layer "F.Cu") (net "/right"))
 (segment (start 48.1 47.8) (end 51.54 51.24) (width 0.2) (layer "F.Cu") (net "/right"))
 (segment (start 53.086346 28.45) (end 53.76 29.123654) (width 0.2) (layer "F.Cu") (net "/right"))
 (via (at 52.2 51.25) (size 0.6) (drill 0.3) (layers "F.Cu" "B.Cu") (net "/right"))
 (segment (start 52.2 58.05) (end 52.2 51.25) (width 0.2) (layer "B.Cu") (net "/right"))
 (segment (start 55.5 61.35) (end 52.2 58.05) (width 0.2) (layer "B.Cu") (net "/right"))
 (segment (start 62 61.35) (end 55.5 61.35) (width 0.2) (layer "B.Cu") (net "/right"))
 (segment (start 38.7 52.15) (end 40.4 53.85) (width 0.2) (layer "F.Cu") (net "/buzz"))
 (segment (start 50 43.375001) (end 50 48.85) (width 0.2) (layer "F.Cu") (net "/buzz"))
 (segment (start 47.7 44.35) (end 49.7 42.35) (width 0.2) (layer "F.Cu") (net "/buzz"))
 (segment (start 52.05 42.35) (end 51.025001 42.35) (width 0.2) (layer "F.Cu") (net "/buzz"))
 (segment (start 51.025001 42.35) (end 50 43.375001) (width 0.2) (layer "F.Cu") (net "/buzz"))
 (segment (start 49.7 42.35) (end 52.05 42.35) (width 0.2) (layer "F.Cu") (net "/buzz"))
 (segment (start 48.6 50.25) (end 45 53.85) (width 0.2) (layer "F.Cu") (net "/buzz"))
 (segment (start 45 53.85) (end 41.8 53.85) (width 0.2) (layer "F.Cu") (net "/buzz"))
 (segment (start 47.7 44.35) (end 47.7 44.9) (width 0.2) (layer "F.Cu") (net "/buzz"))
 (segment (start 36.4 52.15) (end 38.7 52.15) (width 0.2) (layer "F.Cu") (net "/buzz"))
 (via (at 40.4 53.85) (size 0.6) (drill 0.3) (layers "F.Cu" "B.Cu") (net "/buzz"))
 (via (at 50 48.85) (size 0.6) (drill 0.3) (layers "F.Cu" "B.Cu") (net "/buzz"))
 (via (at 48.6 50.25) (size 0.6) (drill 0.3) (layers "F.Cu" "B.Cu") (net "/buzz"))
 (via (at 41.8 53.85) (size 0.6) (drill 0.3) (layers "F.Cu" "B.Cu") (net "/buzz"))
 (segment (start 50 48.85) (end 48.6 50.25) (width 0.2) (layer "B.Cu") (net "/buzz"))
 (segment (start 41.8 53.85) (end 40.4 53.85) (width 0.2) (layer "B.Cu") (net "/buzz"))
 (segment (start 48.3 62.65) (end 52.5 58.45) (width 0.2) (layer "F.Cu") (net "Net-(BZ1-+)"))
 (segment (start 41.561522 62.65) (end 48.3 62.65) (width 0.2) (layer "F.Cu") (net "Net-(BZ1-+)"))
 (segment (start 36.4 54.15) (end 40.7 58.45) (width 0.2) (layer "F.Cu") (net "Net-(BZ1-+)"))
 (segment (start 40.7 61.788478) (end 41.561522 62.65) (width 0.2) (layer "F.Cu") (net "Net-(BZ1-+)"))
 (segment (start 40.7 58.45) (end 40.7 61.788478) (width 0.2) (layer "F.Cu") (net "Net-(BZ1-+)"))
 (segment (start 51.84 45.95) (end 52.05 46.16) (width 0.15) (layer "F.Cu") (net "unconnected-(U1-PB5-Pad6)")))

